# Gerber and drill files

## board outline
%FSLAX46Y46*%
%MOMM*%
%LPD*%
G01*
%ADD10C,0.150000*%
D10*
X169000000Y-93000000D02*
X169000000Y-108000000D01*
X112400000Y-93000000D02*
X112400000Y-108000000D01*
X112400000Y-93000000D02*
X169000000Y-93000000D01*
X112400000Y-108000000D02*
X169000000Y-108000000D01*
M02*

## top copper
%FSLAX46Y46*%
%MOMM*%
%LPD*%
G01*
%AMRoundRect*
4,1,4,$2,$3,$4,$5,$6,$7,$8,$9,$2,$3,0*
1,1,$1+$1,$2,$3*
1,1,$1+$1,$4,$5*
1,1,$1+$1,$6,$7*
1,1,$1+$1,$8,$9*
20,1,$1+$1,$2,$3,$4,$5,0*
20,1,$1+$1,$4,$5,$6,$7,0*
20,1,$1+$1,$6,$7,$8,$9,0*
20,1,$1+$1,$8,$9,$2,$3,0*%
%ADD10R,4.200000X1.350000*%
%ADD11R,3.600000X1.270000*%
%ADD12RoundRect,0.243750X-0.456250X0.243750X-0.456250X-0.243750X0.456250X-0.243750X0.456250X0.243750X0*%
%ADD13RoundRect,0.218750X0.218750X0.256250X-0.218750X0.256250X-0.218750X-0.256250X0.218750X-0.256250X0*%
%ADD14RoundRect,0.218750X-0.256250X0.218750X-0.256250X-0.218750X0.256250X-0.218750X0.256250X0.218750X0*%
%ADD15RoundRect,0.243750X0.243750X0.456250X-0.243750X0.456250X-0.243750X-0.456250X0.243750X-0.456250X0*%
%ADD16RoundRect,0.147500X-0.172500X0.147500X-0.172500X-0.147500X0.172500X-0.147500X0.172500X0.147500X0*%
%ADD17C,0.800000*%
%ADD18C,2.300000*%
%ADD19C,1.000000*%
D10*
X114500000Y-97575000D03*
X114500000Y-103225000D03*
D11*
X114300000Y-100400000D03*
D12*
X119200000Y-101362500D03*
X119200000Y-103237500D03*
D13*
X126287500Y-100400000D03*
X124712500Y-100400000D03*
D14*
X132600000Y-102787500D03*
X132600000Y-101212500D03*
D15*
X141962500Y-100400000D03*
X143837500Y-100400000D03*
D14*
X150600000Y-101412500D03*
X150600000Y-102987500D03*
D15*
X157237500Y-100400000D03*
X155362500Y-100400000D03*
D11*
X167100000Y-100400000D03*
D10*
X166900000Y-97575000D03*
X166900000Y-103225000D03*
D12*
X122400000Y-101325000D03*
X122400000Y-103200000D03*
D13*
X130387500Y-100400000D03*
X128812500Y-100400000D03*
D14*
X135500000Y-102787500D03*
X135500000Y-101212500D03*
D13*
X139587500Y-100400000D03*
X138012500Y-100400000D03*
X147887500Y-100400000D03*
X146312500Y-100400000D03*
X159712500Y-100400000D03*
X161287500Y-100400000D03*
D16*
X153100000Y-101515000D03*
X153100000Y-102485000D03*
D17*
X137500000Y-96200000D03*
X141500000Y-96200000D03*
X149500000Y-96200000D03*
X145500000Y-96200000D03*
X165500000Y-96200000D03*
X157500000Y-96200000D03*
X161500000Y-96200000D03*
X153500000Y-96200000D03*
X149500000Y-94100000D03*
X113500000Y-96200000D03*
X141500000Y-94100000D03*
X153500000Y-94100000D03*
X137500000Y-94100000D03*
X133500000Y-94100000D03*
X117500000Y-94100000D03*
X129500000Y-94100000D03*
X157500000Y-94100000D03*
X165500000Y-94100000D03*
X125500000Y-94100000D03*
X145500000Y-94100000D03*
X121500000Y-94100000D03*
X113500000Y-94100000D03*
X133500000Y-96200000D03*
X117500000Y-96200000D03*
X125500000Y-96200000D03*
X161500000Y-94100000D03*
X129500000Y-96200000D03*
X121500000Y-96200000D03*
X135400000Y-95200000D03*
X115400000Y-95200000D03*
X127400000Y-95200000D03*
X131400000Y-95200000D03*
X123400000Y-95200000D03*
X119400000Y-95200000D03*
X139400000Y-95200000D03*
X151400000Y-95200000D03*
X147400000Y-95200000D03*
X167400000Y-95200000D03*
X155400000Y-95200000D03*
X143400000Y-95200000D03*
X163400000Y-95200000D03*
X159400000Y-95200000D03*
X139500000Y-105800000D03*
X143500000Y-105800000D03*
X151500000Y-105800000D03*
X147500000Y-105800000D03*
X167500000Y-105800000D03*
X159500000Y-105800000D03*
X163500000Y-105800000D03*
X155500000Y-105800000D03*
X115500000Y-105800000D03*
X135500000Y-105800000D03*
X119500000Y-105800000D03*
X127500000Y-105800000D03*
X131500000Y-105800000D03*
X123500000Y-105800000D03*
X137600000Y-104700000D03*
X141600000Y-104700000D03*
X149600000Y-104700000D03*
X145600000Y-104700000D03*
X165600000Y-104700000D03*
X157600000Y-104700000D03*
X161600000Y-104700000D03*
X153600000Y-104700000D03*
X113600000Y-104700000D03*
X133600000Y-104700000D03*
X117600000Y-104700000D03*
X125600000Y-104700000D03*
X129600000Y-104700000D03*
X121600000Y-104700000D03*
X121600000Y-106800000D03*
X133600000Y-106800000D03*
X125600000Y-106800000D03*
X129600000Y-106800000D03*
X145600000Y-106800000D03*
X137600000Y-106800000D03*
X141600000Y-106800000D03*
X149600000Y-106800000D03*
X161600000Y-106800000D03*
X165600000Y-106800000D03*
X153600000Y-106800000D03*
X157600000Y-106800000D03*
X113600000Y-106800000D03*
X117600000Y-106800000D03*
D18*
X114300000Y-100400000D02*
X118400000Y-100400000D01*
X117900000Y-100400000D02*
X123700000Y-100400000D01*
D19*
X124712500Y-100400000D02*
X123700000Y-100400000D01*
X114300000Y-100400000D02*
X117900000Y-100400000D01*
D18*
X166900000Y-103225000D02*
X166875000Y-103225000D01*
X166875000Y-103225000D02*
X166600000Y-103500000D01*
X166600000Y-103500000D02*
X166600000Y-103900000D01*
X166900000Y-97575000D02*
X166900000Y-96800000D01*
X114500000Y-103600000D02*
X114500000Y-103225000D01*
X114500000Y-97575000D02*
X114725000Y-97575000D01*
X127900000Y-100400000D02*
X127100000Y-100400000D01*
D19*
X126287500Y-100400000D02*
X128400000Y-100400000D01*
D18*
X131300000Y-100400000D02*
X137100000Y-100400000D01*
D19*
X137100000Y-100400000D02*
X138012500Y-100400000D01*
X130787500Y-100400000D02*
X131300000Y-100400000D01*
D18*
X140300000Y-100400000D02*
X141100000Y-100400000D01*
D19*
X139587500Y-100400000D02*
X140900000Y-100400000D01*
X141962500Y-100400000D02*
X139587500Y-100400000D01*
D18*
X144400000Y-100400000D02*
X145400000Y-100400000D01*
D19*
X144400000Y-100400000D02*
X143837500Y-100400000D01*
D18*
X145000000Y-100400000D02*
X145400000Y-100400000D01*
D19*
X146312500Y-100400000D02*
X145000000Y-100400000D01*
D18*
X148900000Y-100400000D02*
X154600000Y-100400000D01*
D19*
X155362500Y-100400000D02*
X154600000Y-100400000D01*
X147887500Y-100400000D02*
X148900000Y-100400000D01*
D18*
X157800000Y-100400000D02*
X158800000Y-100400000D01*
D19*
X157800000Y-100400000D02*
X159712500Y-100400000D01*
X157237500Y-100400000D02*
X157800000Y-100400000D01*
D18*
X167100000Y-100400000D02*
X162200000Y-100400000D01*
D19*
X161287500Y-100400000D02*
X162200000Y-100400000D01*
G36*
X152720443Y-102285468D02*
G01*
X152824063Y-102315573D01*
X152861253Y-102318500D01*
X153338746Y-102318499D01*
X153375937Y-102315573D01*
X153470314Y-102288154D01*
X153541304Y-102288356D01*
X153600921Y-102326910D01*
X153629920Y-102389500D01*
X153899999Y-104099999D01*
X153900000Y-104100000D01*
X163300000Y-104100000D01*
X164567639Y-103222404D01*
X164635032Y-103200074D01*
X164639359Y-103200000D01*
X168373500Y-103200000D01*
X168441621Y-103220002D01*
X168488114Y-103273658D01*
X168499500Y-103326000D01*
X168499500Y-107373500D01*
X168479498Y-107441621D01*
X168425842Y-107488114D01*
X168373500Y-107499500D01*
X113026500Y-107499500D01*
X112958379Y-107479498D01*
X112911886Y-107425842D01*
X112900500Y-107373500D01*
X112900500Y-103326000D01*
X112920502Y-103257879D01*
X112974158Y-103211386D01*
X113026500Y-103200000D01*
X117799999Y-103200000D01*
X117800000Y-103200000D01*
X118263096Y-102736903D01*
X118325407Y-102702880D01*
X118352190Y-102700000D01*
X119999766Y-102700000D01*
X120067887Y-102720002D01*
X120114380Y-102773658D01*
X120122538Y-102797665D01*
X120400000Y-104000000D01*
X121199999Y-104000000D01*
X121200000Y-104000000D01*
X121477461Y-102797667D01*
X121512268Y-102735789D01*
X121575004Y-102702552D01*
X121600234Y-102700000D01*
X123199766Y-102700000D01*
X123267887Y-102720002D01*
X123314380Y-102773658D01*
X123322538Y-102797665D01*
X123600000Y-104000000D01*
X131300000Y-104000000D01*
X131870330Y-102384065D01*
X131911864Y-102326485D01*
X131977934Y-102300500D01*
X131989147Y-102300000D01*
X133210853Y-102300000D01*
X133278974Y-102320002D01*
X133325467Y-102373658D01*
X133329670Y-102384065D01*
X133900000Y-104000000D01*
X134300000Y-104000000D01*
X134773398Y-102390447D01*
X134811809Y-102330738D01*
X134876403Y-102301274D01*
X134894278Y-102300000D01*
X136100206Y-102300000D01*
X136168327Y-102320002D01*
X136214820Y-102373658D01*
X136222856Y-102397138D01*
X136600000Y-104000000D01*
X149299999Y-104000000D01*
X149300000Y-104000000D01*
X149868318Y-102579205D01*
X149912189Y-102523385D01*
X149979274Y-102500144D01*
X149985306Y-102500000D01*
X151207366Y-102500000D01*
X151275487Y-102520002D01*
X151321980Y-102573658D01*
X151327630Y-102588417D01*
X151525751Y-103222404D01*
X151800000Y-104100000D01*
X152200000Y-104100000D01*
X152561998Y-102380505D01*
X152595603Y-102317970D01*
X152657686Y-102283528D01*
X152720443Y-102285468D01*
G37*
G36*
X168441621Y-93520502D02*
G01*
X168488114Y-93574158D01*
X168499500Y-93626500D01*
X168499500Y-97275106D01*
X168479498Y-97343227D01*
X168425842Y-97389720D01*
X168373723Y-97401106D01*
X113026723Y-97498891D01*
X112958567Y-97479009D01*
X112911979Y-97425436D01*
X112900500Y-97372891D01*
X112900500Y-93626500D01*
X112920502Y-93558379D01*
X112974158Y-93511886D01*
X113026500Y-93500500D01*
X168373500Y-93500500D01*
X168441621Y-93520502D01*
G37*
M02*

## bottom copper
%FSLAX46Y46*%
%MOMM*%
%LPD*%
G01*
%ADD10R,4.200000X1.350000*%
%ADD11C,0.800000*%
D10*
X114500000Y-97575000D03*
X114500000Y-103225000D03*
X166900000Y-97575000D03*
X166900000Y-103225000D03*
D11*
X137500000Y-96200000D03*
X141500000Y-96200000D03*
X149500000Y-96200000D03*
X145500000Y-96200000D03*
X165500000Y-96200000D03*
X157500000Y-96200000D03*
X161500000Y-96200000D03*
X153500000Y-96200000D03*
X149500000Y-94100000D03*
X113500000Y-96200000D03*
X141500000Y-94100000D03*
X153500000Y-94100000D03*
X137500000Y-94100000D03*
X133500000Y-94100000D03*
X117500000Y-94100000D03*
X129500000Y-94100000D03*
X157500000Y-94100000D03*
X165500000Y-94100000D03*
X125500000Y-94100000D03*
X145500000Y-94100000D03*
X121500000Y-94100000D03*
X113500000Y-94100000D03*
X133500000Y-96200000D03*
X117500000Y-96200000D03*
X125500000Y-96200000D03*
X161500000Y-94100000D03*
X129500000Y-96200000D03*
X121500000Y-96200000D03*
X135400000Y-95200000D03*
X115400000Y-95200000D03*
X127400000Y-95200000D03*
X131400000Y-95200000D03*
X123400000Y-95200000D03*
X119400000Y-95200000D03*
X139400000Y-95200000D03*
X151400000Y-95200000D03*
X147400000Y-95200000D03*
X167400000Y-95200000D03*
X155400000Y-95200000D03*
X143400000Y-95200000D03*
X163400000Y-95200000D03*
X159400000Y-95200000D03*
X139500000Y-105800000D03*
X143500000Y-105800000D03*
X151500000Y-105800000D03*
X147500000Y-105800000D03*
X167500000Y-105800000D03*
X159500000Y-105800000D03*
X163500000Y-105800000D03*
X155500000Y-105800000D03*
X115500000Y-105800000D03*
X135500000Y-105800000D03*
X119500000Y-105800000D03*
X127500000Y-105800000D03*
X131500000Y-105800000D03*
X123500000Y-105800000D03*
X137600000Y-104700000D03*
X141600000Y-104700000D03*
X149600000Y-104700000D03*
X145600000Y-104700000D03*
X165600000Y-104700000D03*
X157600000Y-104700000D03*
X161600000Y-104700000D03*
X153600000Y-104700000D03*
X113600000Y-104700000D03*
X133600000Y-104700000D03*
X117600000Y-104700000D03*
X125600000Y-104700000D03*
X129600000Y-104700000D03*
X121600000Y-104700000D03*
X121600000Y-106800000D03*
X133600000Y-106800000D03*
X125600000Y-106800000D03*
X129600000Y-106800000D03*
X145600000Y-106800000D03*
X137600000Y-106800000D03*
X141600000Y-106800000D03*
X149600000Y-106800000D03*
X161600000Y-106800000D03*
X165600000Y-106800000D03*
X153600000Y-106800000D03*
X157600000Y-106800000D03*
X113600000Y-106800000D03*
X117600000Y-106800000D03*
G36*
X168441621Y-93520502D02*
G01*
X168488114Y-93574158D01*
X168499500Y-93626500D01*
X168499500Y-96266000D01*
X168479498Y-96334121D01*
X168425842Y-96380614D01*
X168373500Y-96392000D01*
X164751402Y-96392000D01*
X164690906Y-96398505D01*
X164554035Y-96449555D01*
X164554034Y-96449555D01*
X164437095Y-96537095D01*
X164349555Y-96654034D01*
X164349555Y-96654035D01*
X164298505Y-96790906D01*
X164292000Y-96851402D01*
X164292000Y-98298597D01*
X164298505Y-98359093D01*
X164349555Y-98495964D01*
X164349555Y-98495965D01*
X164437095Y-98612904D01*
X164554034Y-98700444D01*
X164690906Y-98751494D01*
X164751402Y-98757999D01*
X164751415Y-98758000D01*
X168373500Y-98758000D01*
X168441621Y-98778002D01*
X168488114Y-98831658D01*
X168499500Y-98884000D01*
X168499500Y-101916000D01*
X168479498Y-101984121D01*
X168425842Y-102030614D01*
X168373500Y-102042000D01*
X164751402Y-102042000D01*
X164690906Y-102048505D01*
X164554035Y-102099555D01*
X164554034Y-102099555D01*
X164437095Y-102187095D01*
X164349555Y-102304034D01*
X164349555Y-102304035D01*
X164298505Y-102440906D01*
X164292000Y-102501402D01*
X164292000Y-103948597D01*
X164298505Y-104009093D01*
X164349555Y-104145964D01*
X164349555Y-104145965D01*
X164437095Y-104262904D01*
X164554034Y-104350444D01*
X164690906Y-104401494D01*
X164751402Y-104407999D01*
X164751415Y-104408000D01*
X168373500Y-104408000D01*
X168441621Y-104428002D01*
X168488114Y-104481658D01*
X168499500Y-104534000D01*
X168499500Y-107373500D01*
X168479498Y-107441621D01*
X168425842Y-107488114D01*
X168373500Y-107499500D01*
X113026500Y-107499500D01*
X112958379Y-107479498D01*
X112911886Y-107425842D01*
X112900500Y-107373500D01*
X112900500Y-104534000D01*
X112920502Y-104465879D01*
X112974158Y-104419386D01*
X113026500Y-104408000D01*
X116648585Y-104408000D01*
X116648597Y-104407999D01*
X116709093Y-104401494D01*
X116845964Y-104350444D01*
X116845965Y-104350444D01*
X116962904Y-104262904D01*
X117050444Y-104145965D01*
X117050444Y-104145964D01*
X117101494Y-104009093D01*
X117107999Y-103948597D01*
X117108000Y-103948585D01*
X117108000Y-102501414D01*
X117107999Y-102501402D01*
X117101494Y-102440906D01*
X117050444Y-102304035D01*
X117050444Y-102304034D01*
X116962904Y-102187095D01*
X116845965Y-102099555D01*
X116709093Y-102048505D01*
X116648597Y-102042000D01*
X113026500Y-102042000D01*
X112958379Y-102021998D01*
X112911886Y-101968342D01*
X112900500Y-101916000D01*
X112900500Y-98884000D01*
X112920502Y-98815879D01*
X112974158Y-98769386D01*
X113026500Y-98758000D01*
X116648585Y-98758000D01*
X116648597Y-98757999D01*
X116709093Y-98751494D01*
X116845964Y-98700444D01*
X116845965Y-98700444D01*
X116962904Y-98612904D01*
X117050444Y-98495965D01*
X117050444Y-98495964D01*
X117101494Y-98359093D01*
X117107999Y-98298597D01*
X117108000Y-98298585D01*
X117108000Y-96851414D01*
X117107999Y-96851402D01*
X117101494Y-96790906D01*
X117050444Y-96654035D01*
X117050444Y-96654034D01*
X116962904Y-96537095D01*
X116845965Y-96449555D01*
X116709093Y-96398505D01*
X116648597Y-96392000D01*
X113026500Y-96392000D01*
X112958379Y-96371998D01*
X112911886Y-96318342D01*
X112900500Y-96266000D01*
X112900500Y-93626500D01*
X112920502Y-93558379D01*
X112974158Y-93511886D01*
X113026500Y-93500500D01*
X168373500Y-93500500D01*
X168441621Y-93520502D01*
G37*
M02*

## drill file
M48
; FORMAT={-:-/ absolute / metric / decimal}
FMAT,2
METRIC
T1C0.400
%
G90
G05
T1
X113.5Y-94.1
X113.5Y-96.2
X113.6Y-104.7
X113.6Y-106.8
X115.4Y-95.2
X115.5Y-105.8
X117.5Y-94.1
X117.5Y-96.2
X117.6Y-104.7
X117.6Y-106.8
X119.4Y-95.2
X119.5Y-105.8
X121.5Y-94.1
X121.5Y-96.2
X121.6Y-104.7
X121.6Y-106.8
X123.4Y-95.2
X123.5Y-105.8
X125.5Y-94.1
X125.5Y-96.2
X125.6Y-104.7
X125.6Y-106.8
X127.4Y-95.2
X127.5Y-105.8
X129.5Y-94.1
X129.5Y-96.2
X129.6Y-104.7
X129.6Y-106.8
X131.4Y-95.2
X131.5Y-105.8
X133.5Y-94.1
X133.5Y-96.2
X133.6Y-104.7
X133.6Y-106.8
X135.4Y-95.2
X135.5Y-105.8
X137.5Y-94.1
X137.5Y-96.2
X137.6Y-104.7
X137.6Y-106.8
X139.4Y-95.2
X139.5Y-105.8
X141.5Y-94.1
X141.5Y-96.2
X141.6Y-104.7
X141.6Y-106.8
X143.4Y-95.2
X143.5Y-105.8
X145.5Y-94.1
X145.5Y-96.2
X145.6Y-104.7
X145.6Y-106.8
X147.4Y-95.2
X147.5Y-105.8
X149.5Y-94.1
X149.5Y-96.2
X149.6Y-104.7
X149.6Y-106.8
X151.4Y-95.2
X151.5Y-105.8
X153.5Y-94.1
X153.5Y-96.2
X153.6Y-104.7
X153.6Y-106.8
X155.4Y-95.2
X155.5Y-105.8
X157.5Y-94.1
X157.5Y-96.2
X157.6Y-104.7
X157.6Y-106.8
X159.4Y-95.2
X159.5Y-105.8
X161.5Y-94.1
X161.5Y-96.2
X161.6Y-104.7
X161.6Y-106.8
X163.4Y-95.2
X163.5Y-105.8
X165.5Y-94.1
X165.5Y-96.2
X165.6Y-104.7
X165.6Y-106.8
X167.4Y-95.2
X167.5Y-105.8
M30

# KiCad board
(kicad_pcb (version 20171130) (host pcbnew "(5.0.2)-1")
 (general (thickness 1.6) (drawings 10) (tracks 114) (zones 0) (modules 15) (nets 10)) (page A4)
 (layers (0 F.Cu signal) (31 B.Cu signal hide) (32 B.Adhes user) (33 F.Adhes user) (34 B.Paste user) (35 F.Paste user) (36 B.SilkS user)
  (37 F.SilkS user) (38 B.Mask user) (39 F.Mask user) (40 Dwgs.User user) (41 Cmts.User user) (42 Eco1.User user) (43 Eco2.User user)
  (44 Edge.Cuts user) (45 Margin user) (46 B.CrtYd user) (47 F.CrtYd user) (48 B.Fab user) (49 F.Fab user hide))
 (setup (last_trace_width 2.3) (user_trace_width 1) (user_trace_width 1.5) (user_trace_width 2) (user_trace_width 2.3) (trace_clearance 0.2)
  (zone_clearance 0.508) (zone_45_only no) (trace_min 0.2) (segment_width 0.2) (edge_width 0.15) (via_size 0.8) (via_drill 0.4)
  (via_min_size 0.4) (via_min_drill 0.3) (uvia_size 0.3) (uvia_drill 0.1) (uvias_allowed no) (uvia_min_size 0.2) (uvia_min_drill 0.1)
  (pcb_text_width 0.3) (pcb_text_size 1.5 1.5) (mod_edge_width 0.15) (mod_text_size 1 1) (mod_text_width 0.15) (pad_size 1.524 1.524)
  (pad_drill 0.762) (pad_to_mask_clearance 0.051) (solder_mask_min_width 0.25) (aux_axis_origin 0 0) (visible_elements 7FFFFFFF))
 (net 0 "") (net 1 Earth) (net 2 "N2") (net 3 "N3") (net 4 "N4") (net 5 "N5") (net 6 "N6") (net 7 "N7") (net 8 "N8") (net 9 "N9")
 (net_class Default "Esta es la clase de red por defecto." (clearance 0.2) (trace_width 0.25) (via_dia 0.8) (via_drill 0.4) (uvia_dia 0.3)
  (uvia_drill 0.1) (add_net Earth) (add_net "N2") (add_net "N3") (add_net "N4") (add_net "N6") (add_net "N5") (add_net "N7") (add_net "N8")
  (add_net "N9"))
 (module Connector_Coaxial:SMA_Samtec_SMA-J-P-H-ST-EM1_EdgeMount (layer F.Cu) (at 114.5 100.4 180)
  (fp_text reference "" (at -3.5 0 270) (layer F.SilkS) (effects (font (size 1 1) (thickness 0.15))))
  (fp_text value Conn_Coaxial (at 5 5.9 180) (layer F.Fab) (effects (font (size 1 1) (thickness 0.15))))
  (pad 2 smd rect (at 0 2.825 270) (size 1.35 4.2) (layers B.Cu B.Paste B.Mask) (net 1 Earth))
  (pad 2 smd rect (at 0 -2.825 270) (size 1.35 4.2) (layers B.Cu B.Paste B.Mask) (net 1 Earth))
  (pad 2 smd rect (at 0 2.825 270) (size 1.35 4.2) (layers F.Cu F.Paste F.Mask) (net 1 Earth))
  (pad 2 smd rect (at 0 -2.825 270) (size 1.35 4.2) (layers F.Cu F.Paste F.Mask) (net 1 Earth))
  (pad 1 smd rect (at 0.2 0 270) (size 1.27 3.6) (layers F.Cu F.Paste F.Mask) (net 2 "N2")))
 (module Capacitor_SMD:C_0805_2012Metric (layer F.Cu) (at 119.2 102.3 270)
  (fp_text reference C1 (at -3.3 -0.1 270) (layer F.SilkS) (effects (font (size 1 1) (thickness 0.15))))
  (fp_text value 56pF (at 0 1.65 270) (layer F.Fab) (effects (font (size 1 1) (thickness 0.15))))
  (pad 1 smd roundrect (at -0.9375 0 270) (size 0.975 1.4) (layers F.Cu F.Paste F.Mask) (roundrect_rratio 0.25) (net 2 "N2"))
  (pad 2 smd roundrect (at 0.9375 0 270) (size 0.975 1.4) (layers F.Cu F.Paste F.Mask) (roundrect_rratio 0.25) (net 1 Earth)))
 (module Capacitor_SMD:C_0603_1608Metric (layer F.Cu) (at 125.5 100.4 180)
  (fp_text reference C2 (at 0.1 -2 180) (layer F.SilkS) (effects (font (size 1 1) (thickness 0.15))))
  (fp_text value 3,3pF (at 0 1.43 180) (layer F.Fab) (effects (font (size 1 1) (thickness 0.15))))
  (pad 1 smd roundrect (at -0.7875 0 180) (size 0.875 0.95) (layers F.Cu F.Paste F.Mask) (roundrect_rratio 0.25) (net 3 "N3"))
  (pad 2 smd roundrect (at 0.7875 0 180) (size 0.875 0.95) (layers F.Cu F.Paste F.Mask) (roundrect_rratio 0.25) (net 2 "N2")))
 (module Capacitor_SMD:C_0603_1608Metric (layer F.Cu) (at 132.6 102 270)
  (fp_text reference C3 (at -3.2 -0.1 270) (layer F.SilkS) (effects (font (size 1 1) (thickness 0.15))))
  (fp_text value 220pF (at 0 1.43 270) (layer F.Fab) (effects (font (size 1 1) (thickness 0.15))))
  (pad 2 smd roundrect (at 0.7875 0 270) (size 0.875 0.95) (layers F.Cu F.Paste F.Mask) (roundrect_rratio 0.25) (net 1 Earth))
  (pad 1 smd roundrect (at -0.7875 0 270) (size 0.875 0.95) (layers F.Cu F.Paste F.Mask) (roundrect_rratio 0.25) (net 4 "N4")))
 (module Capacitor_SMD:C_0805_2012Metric (layer F.Cu) (at 142.9 100.4 180)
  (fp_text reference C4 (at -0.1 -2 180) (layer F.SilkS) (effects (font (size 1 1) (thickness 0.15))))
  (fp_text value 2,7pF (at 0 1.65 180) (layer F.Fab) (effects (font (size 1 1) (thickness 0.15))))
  (pad 2 smd roundrect (at 0.9375 0 180) (size 0.975 1.4) (layers F.Cu F.Paste F.Mask) (roundrect_rratio 0.25) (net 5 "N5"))
  (pad 1 smd roundrect (at -0.9375 0 180) (size 0.975 1.4) (layers F.Cu F.Paste F.Mask) (roundrect_rratio 0.25) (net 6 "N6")))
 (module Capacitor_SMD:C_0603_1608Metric (layer F.Cu) (at 150.6 102.2 270)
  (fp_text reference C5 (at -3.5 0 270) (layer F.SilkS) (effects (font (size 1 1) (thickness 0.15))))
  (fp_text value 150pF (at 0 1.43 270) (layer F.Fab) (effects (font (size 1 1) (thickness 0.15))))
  (pad 1 smd roundrect (at -0.7875 0 270) (size 0.875 0.95) (layers F.Cu F.Paste F.Mask) (roundrect_rratio 0.25) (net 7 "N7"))
  (pad 2 smd roundrect (at 0.7875 0 270) (size 0.875 0.95) (layers F.Cu F.Paste F.Mask) (roundrect_rratio 0.25) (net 1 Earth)))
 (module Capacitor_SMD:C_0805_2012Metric (layer F.Cu) (at 156.3 100.4 180)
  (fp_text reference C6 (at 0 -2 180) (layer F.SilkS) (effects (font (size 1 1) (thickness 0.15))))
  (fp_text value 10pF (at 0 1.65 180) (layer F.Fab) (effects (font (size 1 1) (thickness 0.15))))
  (pad 1 smd roundrect (at -0.9375 0 180) (size 0.975 1.4) (layers F.Cu F.Paste F.Mask) (roundrect_rratio 0.25) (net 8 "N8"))
  (pad 2 smd roundrect (at 0.9375 0 180) (size 0.975 1.4) (layers F.Cu F.Paste F.Mask) (roundrect_rratio 0.25) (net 7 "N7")))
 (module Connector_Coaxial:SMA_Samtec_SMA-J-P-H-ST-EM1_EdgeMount (layer F.Cu) (at 166.9 100.4)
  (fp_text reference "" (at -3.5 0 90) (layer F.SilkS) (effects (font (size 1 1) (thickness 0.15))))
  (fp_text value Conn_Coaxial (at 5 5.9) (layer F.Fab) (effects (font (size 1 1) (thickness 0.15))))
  (pad 1 smd rect (at 0.2 0 90) (size 1.27 3.6) (layers F.Cu F.Paste F.Mask) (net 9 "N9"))
  (pad 2 smd rect (at 0 -2.825 90) (size 1.35 4.2) (layers F.Cu F.Paste F.Mask) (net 1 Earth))
  (pad 2 smd rect (at 0 2.825 90) (size 1.35 4.2) (layers F.Cu F.Paste F.Mask) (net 1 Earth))
  (pad 2 smd rect (at 0 -2.825 90) (size 1.35 4.2) (layers B.Cu B.Paste B.Mask) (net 1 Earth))
  (pad 2 smd rect (at 0 2.825 90) (size 1.35 4.2) (layers B.Cu B.Paste B.Mask) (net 1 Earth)))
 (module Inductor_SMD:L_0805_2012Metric (layer F.Cu) (at 122.4 102.2625 270)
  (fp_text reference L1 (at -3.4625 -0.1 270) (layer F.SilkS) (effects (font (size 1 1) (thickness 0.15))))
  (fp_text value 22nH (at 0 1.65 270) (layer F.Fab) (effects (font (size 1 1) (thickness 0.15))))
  (pad 1 smd roundrect (at -0.9375 0 270) (size 0.975 1.4) (layers F.Cu F.Paste F.Mask) (roundrect_rratio 0.25) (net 2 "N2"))
  (pad 2 smd roundrect (at 0.9375 0 270) (size 0.975 1.4) (layers F.Cu F.Paste F.Mask) (roundrect_rratio 0.25) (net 1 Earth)))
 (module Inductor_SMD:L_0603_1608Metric (layer F.Cu) (at 129.6 100.4 180)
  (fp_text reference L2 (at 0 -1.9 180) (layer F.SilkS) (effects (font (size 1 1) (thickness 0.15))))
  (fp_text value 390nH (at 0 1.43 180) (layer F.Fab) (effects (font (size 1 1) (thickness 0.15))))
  (pad 1 smd roundrect (at -0.7875 0 180) (size 0.875 0.95) (layers F.Cu F.Paste F.Mask) (roundrect_rratio 0.25) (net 4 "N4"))
  (pad 2 smd roundrect (at 0.7875 0 180) (size 0.875 0.95) (layers F.Cu F.Paste F.Mask) (roundrect_rratio 0.25) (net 3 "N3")))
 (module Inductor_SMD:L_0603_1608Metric (layer F.Cu) (at 135.5 102 270)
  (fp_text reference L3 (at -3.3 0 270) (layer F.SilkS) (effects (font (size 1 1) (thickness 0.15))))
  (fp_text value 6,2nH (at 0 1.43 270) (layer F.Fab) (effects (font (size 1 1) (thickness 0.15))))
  (pad 2 smd roundrect (at 0.7875 0 270) (size 0.875 0.95) (layers F.Cu F.Paste F.Mask) (roundrect_rratio 0.25) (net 1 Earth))
  (pad 1 smd roundrect (at -0.7875 0 270) (size 0.875 0.95) (layers F.Cu F.Paste F.Mask) (roundrect_rratio 0.25) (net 4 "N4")))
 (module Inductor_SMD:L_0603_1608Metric (layer F.Cu) (at 138.8 100.4 180)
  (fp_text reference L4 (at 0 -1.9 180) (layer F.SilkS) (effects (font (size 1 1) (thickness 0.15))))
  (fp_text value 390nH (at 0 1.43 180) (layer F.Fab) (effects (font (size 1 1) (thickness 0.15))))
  (pad 1 smd roundrect (at -0.7875 0 180) (size 0.875 0.95) (layers F.Cu F.Paste F.Mask) (roundrect_rratio 0.25) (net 5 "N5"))
  (pad 2 smd roundrect (at 0.7875 0 180) (size 0.875 0.95) (layers F.Cu F.Paste F.Mask) (roundrect_rratio 0.25) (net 4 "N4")))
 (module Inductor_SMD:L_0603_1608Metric (layer F.Cu) (at 147.1 100.4 180)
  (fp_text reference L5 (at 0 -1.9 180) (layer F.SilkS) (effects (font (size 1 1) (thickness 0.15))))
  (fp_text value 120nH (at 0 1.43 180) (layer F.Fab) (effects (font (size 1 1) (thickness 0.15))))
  (pad 1 smd roundrect (at -0.7875 0 180) (size 0.875 0.95) (layers F.Cu F.Paste F.Mask) (roundrect_rratio 0.25) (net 7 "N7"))
  (pad 2 smd roundrect (at 0.7875 0 180) (size 0.875 0.95) (layers F.Cu F.Paste F.Mask) (roundrect_rratio 0.25) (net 6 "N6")))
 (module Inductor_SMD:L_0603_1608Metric (layer F.Cu) (at 160.5 100.4 180)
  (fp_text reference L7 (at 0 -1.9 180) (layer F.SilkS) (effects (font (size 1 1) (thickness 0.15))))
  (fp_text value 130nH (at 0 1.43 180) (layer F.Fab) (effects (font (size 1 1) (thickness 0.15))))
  (pad 2 smd roundrect (at 0.7875 0 180) (size 0.875 0.95) (layers F.Cu F.Paste F.Mask) (roundrect_rratio 0.25) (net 8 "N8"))
  (pad 1 smd roundrect (at -0.7875 0 180) (size 0.875 0.95) (layers F.Cu F.Paste F.Mask) (roundrect_rratio 0.25) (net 9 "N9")))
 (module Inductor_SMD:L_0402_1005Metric (layer F.Cu) (at 153.1 102 270)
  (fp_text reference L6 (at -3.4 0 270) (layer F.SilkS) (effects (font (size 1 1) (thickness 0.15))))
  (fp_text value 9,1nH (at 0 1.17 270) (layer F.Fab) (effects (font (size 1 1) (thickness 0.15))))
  (pad 1 smd roundrect (at -0.485 0 270) (size 0.59 0.64) (layers F.Cu F.Paste F.Mask) (roundrect_rratio 0.25) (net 7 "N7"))
  (pad 2 smd roundrect (at 0.485 0 270) (size 0.59 0.64) (layers F.Cu F.Paste F.Mask) (roundrect_rratio 0.25) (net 1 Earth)))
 (gr_line (start 169 93) (end 169 108) (layer Edge.Cuts) (width 0.15))
 (gr_line (start 112.4 93) (end 112.4 108) (layer Edge.Cuts) (width 0.15))
 (gr_line (start 112.4 93) (end 169 93) (layer Edge.Cuts) (width 0.15))
 (gr_line (start 112.4 108) (end 169 108) (layer Edge.Cuts) (width 0.15))
 (via (at 137.5 96.2) (size 0.8) (drill 0.4) (layers F.Cu B.Cu) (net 1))
 (via (at 141.5 96.2) (size 0.8) (drill 0.4) (layers F.Cu B.Cu) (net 1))
 (via (at 149.5 96.2) (size 0.8) (drill 0.4) (layers F.Cu B.Cu) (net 1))
 (via (at 145.5 96.2) (size 0.8) (drill 0.4) (layers F.Cu B.Cu) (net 1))
 (via (at 165.5 96.2) (size 0.8) (drill 0.4) (layers F.Cu B.Cu) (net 1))
 (via (at 157.5 96.2) (size 0.8) (drill 0.4) (layers F.Cu B.Cu) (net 1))
 (via (at 161.5 96.2) (size 0.8) (drill 0.4) (layers F.Cu B.Cu) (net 1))
 (via (at 153.5 96.2) (size 0.8) (drill 0.4) (layers F.Cu B.Cu) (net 1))
 (via (at 149.5 94.1) (size 0.8) (drill 0.4) (layers F.Cu B.Cu) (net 1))
 (via (at 113.5 96.2) (size 0.8) (drill 0.4) (layers F.Cu B.Cu) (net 1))
 (via (at 141.5 94.1) (size 0.8) (drill 0.4) (layers F.Cu B.Cu) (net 1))
 (via (at 153.5 94.1) (size 0.8) (drill 0.4) (layers F.Cu B.Cu) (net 1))
 (via (at 137.5 94.1) (size 0.8) (drill 0.4) (layers F.Cu B.Cu) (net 1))
 (via (at 133.5 94.1) (size 0.8) (drill 0.4) (layers F.Cu B.Cu) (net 1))
 (via (at 117.5 94.1) (size 0.8) (drill 0.4) (layers F.Cu B.Cu) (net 1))
 (via (at 129.5 94.1) (size 0.8) (drill 0.4) (layers F.Cu B.Cu) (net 1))
 (via (at 157.5 94.1) (size 0.8) (drill 0.4) (layers F.Cu B.Cu) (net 1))
 (via (at 165.5 94.1) (size 0.8) (drill 0.4) (layers F.Cu B.Cu) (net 1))
 (via (at 125.5 94.1) (size 0.8) (drill 0.4) (layers F.Cu B.Cu) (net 1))
 (via (at 145.5 94.1) (size 0.8) (drill 0.4) (layers F.Cu B.Cu) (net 1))
 (via (at 121.5 94.1) (size 0.8) (drill 0.4) (layers F.Cu B.Cu) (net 1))
 (via (at 113.5 94.1) (size 0.8) (drill 0.4) (layers F.Cu B.Cu) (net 1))
 (via (at 133.5 96.2) (size 0.8) (drill 0.4) (layers F.Cu B.Cu) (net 1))
 (via (at 117.5 96.2) (size 0.8) (drill 0.4) (layers F.Cu B.Cu) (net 1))
 (via (at 125.5 96.2) (size 0.8) (drill 0.4) (layers F.Cu B.Cu) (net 1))
 (via (at 161.5 94.1) (size 0.8) (drill 0.4) (layers F.Cu B.Cu) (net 1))
 (via (at 129.5 96.2) (size 0.8) (drill 0.4) (layers F.Cu B.Cu) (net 1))
 (via (at 121.5 96.2) (size 0.8) (drill 0.4) (layers F.Cu B.Cu) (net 1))
 (via (at 135.4 95.2) (size 0.8) (drill 0.4) (layers F.Cu B.Cu) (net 1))
 (via (at 115.4 95.2) (size 0.8) (drill 0.4) (layers F.Cu B.Cu) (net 1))
 (via (at 127.4 95.2) (size 0.8) (drill 0.4) (layers F.Cu B.Cu) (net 1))
 (via (at 131.4 95.2) (size 0.8) (drill 0.4) (layers F.Cu B.Cu) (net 1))
 (via (at 123.4 95.2) (size 0.8) (drill 0.4) (layers F.Cu B.Cu) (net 1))
 (via (at 119.4 95.2) (size 0.8) (drill 0.4) (layers F.Cu B.Cu) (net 1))
 (via (at 139.4 95.2) (size 0.8) (drill 0.4) (layers F.Cu B.Cu) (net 1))
 (via (at 151.4 95.2) (size 0.8) (drill 0.4) (layers F.Cu B.Cu) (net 1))
 (via (at 147.4 95.2) (size 0.8) (drill 0.4) (layers F.Cu B.Cu) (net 1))
 (via (at 167.4 95.2) (size 0.8) (drill 0.4) (layers F.Cu B.Cu) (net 1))
 (via (at 155.4 95.2) (size 0.8) (drill 0.4) (layers F.Cu B.Cu) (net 1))
 (via (at 143.4 95.2) (size 0.8) (drill 0.4) (layers F.Cu B.Cu) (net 1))
 (via (at 163.4 95.2) (size 0.8) (drill 0.4) (layers F.Cu B.Cu) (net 1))
 (via (at 159.4 95.2) (size 0.8) (drill 0.4) (layers F.Cu B.Cu) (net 1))
 (via (at 139.5 105.8) (size 0.8) (drill 0.4) (layers F.Cu B.Cu) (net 1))
 (via (at 143.5 105.8) (size 0.8) (drill 0.4) (layers F.Cu B.Cu) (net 1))
 (via (at 151.5 105.8) (size 0.8) (drill 0.4) (layers F.Cu B.Cu) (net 1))
 (via (at 147.5 105.8) (size 0.8) (drill 0.4) (layers F.Cu B.Cu) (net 1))
 (via (at 167.5 105.8) (size 0.8) (drill 0.4) (layers F.Cu B.Cu) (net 1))
 (via (at 159.5 105.8) (size 0.8) (drill 0.4) (layers F.Cu B.Cu) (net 1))
 (via (at 163.5 105.8) (size 0.8) (drill 0.4) (layers F.Cu B.Cu) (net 1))
 (via (at 155.5 105.8) (size 0.8) (drill 0.4) (layers F.Cu B.Cu) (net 1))
 (via (at 115.5 105.8) (size 0.8) (drill 0.4) (layers F.Cu B.Cu) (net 1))
 (via (at 135.5 105.8) (size 0.8) (drill 0.4) (layers F.Cu B.Cu) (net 1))
 (via (at 119.5 105.8) (size 0.8) (drill 0.4) (layers F.Cu B.Cu) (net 1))
 (via (at 127.5 105.8) (size 0.8) (drill 0.4) (layers F.Cu B.Cu) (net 1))
 (via (at 131.5 105.8) (size 0.8) (drill 0.4) (layers F.Cu B.Cu) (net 1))
 (via (at 123.5 105.8) (size 0.8) (drill 0.4) (layers F.Cu B.Cu) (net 1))
 (via (at 137.6 104.7) (size 0.8) (drill 0.4) (layers F.Cu B.Cu) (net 1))
 (via (at 141.6 104.7) (size 0.8) (drill 0.4) (layers F.Cu B.Cu) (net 1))
 (via (at 149.6 104.7) (size 0.8) (drill 0.4) (layers F.Cu B.Cu) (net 1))
 (via (at 145.6 104.7) (size 0.8) (drill 0.4) (layers F.Cu B.Cu) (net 1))
 (via (at 165.6 104.7) (size 0.8) (drill 0.4) (layers F.Cu B.Cu) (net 1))
 (via (at 157.6 104.7) (size 0.8) (drill 0.4) (layers F.Cu B.Cu) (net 1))
 (via (at 161.6 104.7) (size 0.8) (drill 0.4) (layers F.Cu B.Cu) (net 1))
 (via (at 153.6 104.7) (size 0.8) (drill 0.4) (layers F.Cu B.Cu) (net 1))
 (via (at 113.6 104.7) (size 0.8) (drill 0.4) (layers F.Cu B.Cu) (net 1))
 (via (at 133.6 104.7) (size 0.8) (drill 0.4) (layers F.Cu B.Cu) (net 1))
 (via (at 117.6 104.7) (size 0.8) (drill 0.4) (layers F.Cu B.Cu) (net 1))
 (via (at 125.6 104.7) (size 0.8) (drill 0.4) (layers F.Cu B.Cu) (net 1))
 (via (at 129.6 104.7) (size 0.8) (drill 0.4) (layers F.Cu B.Cu) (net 1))
 (via (at 121.6 104.7) (size 0.8) (drill 0.4) (layers F.Cu B.Cu) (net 1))
 (via (at 121.6 106.8) (size 0.8) (drill 0.4) (layers F.Cu B.Cu) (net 1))
 (via (at 133.6 106.8) (size 0.8) (drill 0.4) (layers F.Cu B.Cu) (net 1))
 (via (at 125.6 106.8) (size 0.8) (drill 0.4) (layers F.Cu B.Cu) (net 1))
 (via (at 129.6 106.8) (size 0.8) (drill 0.4) (layers F.Cu B.Cu) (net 1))
 (via (at 145.6 106.8) (size 0.8) (drill 0.4) (layers F.Cu B.Cu) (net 1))
 (via (at 137.6 106.8) (size 0.8) (drill 0.4) (layers F.Cu B.Cu) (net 1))
 (via (at 141.6 106.8) (size 0.8) (drill 0.4) (layers F.Cu B.Cu) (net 1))
 (via (at 149.6 106.8) (size 0.8) (drill 0.4) (layers F.Cu B.Cu) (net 1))
 (via (at 161.6 106.8) (size 0.8) (drill 0.4) (layers F.Cu B.Cu) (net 1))
 (via (at 165.6 106.8) (size 0.8) (drill 0.4) (layers F.Cu B.Cu) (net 1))
 (via (at 153.6 106.8) (size 0.8) (drill 0.4) (layers F.Cu B.Cu) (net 1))
 (via (at 157.6 106.8) (size 0.8) (drill 0.4) (layers F.Cu B.Cu) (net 1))
 (segment (start 114.3 100.4) (end 118.4 100.4) (width 2.3) (layer F.Cu) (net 2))
 (segment (start 117.9 100.4) (end 123.7 100.4) (width 2.3) (layer F.Cu) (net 2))
 (segment (start 124.7125 100.4) (end 123.7 100.4) (width 1) (layer F.Cu) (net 2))
 (segment (start 114.3 100.4) (end 117.9 100.4) (width 1) (layer F.Cu) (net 2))
 (via (at 113.6 106.8) (size 0.8) (drill 0.4) (layers F.Cu B.Cu) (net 1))
 (via (at 117.6 106.8) (size 0.8) (drill 0.4) (layers F.Cu B.Cu) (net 1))
 (segment (start 166.9 103.225) (end 166.875 103.225) (width 2.3) (layer F.Cu) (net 1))
 (segment (start 166.875 103.225) (end 166.6 103.5) (width 2.3) (layer F.Cu) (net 1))
 (segment (start 166.6 103.5) (end 166.6 103.9) (width 2.3) (layer F.Cu) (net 1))
 (segment (start 166.9 97.575) (end 166.9 96.8) (width 2.3) (layer F.Cu) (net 1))
 (segment (start 114.5 103.6) (end 114.5 103.225) (width 2.3) (layer F.Cu) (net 1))
 (segment (start 114.5 97.575) (end 114.725 97.575) (width 2.3) (layer F.Cu) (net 1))
 (segment (start 127.9 100.4) (end 127.1 100.4) (width 2.3) (layer F.Cu) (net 3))
 (segment (start 126.2875 100.4) (end 128.4 100.4) (width 1) (layer F.Cu) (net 3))
 (segment (start 131.3 100.4) (end 137.1 100.4) (width 2.3) (layer F.Cu) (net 4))
 (segment (start 137.1 100.4) (end 138.0125 100.4) (width 1) (layer F.Cu) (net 4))
 (segment (start 130.7875 100.4) (end 131.3 100.4) (width 1) (layer F.Cu) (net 4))
 (segment (start 140.3 100.4) (end 141.1 100.4) (width 2.3) (layer F.Cu) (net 5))
 (segment (start 139.5875 100.4) (end 140.9 100.4) (width 1) (layer F.Cu) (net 5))
 (segment (start 141.9625 100.4) (end 139.5875 100.4) (width 1) (layer F.Cu) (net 5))
 (segment (start 144.4 100.4) (end 145.4 100.4) (width 2.3) (layer F.Cu) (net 6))
 (segment (start 144.4 100.4) (end 143.8375 100.4) (width 1) (layer F.Cu) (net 6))
 (segment (start 145 100.4) (end 145.4 100.4) (width 2.3) (layer F.Cu) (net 6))
 (segment (start 146.3125 100.4) (end 145 100.4) (width 1) (layer F.Cu) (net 6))
 (segment (start 148.9 100.4) (end 154.6 100.4) (width 2.3) (layer F.Cu) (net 7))
 (segment (start 155.3625 100.4) (end 154.6 100.4) (width 1) (layer F.Cu) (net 7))
 (segment (start 147.8875 100.4) (end 148.9 100.4) (width 1) (layer F.Cu) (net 7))
 (segment (start 157.8 100.4) (end 158.8 100.4) (width 2.3) (layer F.Cu) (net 8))
 (segment (start 157.8 100.4) (end 159.7125 100.4) (width 1) (layer F.Cu) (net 8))
 (segment (start 157.2375 100.4) (end 157.8 100.4) (width 1) (layer F.Cu) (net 8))
 (segment (start 167.1 100.4) (end 162.2 100.4) (width 2.3) (layer F.Cu) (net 9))
 (segment (start 161.2875 100.4) (end 162.2 100.4) (width 1) (layer F.Cu) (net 9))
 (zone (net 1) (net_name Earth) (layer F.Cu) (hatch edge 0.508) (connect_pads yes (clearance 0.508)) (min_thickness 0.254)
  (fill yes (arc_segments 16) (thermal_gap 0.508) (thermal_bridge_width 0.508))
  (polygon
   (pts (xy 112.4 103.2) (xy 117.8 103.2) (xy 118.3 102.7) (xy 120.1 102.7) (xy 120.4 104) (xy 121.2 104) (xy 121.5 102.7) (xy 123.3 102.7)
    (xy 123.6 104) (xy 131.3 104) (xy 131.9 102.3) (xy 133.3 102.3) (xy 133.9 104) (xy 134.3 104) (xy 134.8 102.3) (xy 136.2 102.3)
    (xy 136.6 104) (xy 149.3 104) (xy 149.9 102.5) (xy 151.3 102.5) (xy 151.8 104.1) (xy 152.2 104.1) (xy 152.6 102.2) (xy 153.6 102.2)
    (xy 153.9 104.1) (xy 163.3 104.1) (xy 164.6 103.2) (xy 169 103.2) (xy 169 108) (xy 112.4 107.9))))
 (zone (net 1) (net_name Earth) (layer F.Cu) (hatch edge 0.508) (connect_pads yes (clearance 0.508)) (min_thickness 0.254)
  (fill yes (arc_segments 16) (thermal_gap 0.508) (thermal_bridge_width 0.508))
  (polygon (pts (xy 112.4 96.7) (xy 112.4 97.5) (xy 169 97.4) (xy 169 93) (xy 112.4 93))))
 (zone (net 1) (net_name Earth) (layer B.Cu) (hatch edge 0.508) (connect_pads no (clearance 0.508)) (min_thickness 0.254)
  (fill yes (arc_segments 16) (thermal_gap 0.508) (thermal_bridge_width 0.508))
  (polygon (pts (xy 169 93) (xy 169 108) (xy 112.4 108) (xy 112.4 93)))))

